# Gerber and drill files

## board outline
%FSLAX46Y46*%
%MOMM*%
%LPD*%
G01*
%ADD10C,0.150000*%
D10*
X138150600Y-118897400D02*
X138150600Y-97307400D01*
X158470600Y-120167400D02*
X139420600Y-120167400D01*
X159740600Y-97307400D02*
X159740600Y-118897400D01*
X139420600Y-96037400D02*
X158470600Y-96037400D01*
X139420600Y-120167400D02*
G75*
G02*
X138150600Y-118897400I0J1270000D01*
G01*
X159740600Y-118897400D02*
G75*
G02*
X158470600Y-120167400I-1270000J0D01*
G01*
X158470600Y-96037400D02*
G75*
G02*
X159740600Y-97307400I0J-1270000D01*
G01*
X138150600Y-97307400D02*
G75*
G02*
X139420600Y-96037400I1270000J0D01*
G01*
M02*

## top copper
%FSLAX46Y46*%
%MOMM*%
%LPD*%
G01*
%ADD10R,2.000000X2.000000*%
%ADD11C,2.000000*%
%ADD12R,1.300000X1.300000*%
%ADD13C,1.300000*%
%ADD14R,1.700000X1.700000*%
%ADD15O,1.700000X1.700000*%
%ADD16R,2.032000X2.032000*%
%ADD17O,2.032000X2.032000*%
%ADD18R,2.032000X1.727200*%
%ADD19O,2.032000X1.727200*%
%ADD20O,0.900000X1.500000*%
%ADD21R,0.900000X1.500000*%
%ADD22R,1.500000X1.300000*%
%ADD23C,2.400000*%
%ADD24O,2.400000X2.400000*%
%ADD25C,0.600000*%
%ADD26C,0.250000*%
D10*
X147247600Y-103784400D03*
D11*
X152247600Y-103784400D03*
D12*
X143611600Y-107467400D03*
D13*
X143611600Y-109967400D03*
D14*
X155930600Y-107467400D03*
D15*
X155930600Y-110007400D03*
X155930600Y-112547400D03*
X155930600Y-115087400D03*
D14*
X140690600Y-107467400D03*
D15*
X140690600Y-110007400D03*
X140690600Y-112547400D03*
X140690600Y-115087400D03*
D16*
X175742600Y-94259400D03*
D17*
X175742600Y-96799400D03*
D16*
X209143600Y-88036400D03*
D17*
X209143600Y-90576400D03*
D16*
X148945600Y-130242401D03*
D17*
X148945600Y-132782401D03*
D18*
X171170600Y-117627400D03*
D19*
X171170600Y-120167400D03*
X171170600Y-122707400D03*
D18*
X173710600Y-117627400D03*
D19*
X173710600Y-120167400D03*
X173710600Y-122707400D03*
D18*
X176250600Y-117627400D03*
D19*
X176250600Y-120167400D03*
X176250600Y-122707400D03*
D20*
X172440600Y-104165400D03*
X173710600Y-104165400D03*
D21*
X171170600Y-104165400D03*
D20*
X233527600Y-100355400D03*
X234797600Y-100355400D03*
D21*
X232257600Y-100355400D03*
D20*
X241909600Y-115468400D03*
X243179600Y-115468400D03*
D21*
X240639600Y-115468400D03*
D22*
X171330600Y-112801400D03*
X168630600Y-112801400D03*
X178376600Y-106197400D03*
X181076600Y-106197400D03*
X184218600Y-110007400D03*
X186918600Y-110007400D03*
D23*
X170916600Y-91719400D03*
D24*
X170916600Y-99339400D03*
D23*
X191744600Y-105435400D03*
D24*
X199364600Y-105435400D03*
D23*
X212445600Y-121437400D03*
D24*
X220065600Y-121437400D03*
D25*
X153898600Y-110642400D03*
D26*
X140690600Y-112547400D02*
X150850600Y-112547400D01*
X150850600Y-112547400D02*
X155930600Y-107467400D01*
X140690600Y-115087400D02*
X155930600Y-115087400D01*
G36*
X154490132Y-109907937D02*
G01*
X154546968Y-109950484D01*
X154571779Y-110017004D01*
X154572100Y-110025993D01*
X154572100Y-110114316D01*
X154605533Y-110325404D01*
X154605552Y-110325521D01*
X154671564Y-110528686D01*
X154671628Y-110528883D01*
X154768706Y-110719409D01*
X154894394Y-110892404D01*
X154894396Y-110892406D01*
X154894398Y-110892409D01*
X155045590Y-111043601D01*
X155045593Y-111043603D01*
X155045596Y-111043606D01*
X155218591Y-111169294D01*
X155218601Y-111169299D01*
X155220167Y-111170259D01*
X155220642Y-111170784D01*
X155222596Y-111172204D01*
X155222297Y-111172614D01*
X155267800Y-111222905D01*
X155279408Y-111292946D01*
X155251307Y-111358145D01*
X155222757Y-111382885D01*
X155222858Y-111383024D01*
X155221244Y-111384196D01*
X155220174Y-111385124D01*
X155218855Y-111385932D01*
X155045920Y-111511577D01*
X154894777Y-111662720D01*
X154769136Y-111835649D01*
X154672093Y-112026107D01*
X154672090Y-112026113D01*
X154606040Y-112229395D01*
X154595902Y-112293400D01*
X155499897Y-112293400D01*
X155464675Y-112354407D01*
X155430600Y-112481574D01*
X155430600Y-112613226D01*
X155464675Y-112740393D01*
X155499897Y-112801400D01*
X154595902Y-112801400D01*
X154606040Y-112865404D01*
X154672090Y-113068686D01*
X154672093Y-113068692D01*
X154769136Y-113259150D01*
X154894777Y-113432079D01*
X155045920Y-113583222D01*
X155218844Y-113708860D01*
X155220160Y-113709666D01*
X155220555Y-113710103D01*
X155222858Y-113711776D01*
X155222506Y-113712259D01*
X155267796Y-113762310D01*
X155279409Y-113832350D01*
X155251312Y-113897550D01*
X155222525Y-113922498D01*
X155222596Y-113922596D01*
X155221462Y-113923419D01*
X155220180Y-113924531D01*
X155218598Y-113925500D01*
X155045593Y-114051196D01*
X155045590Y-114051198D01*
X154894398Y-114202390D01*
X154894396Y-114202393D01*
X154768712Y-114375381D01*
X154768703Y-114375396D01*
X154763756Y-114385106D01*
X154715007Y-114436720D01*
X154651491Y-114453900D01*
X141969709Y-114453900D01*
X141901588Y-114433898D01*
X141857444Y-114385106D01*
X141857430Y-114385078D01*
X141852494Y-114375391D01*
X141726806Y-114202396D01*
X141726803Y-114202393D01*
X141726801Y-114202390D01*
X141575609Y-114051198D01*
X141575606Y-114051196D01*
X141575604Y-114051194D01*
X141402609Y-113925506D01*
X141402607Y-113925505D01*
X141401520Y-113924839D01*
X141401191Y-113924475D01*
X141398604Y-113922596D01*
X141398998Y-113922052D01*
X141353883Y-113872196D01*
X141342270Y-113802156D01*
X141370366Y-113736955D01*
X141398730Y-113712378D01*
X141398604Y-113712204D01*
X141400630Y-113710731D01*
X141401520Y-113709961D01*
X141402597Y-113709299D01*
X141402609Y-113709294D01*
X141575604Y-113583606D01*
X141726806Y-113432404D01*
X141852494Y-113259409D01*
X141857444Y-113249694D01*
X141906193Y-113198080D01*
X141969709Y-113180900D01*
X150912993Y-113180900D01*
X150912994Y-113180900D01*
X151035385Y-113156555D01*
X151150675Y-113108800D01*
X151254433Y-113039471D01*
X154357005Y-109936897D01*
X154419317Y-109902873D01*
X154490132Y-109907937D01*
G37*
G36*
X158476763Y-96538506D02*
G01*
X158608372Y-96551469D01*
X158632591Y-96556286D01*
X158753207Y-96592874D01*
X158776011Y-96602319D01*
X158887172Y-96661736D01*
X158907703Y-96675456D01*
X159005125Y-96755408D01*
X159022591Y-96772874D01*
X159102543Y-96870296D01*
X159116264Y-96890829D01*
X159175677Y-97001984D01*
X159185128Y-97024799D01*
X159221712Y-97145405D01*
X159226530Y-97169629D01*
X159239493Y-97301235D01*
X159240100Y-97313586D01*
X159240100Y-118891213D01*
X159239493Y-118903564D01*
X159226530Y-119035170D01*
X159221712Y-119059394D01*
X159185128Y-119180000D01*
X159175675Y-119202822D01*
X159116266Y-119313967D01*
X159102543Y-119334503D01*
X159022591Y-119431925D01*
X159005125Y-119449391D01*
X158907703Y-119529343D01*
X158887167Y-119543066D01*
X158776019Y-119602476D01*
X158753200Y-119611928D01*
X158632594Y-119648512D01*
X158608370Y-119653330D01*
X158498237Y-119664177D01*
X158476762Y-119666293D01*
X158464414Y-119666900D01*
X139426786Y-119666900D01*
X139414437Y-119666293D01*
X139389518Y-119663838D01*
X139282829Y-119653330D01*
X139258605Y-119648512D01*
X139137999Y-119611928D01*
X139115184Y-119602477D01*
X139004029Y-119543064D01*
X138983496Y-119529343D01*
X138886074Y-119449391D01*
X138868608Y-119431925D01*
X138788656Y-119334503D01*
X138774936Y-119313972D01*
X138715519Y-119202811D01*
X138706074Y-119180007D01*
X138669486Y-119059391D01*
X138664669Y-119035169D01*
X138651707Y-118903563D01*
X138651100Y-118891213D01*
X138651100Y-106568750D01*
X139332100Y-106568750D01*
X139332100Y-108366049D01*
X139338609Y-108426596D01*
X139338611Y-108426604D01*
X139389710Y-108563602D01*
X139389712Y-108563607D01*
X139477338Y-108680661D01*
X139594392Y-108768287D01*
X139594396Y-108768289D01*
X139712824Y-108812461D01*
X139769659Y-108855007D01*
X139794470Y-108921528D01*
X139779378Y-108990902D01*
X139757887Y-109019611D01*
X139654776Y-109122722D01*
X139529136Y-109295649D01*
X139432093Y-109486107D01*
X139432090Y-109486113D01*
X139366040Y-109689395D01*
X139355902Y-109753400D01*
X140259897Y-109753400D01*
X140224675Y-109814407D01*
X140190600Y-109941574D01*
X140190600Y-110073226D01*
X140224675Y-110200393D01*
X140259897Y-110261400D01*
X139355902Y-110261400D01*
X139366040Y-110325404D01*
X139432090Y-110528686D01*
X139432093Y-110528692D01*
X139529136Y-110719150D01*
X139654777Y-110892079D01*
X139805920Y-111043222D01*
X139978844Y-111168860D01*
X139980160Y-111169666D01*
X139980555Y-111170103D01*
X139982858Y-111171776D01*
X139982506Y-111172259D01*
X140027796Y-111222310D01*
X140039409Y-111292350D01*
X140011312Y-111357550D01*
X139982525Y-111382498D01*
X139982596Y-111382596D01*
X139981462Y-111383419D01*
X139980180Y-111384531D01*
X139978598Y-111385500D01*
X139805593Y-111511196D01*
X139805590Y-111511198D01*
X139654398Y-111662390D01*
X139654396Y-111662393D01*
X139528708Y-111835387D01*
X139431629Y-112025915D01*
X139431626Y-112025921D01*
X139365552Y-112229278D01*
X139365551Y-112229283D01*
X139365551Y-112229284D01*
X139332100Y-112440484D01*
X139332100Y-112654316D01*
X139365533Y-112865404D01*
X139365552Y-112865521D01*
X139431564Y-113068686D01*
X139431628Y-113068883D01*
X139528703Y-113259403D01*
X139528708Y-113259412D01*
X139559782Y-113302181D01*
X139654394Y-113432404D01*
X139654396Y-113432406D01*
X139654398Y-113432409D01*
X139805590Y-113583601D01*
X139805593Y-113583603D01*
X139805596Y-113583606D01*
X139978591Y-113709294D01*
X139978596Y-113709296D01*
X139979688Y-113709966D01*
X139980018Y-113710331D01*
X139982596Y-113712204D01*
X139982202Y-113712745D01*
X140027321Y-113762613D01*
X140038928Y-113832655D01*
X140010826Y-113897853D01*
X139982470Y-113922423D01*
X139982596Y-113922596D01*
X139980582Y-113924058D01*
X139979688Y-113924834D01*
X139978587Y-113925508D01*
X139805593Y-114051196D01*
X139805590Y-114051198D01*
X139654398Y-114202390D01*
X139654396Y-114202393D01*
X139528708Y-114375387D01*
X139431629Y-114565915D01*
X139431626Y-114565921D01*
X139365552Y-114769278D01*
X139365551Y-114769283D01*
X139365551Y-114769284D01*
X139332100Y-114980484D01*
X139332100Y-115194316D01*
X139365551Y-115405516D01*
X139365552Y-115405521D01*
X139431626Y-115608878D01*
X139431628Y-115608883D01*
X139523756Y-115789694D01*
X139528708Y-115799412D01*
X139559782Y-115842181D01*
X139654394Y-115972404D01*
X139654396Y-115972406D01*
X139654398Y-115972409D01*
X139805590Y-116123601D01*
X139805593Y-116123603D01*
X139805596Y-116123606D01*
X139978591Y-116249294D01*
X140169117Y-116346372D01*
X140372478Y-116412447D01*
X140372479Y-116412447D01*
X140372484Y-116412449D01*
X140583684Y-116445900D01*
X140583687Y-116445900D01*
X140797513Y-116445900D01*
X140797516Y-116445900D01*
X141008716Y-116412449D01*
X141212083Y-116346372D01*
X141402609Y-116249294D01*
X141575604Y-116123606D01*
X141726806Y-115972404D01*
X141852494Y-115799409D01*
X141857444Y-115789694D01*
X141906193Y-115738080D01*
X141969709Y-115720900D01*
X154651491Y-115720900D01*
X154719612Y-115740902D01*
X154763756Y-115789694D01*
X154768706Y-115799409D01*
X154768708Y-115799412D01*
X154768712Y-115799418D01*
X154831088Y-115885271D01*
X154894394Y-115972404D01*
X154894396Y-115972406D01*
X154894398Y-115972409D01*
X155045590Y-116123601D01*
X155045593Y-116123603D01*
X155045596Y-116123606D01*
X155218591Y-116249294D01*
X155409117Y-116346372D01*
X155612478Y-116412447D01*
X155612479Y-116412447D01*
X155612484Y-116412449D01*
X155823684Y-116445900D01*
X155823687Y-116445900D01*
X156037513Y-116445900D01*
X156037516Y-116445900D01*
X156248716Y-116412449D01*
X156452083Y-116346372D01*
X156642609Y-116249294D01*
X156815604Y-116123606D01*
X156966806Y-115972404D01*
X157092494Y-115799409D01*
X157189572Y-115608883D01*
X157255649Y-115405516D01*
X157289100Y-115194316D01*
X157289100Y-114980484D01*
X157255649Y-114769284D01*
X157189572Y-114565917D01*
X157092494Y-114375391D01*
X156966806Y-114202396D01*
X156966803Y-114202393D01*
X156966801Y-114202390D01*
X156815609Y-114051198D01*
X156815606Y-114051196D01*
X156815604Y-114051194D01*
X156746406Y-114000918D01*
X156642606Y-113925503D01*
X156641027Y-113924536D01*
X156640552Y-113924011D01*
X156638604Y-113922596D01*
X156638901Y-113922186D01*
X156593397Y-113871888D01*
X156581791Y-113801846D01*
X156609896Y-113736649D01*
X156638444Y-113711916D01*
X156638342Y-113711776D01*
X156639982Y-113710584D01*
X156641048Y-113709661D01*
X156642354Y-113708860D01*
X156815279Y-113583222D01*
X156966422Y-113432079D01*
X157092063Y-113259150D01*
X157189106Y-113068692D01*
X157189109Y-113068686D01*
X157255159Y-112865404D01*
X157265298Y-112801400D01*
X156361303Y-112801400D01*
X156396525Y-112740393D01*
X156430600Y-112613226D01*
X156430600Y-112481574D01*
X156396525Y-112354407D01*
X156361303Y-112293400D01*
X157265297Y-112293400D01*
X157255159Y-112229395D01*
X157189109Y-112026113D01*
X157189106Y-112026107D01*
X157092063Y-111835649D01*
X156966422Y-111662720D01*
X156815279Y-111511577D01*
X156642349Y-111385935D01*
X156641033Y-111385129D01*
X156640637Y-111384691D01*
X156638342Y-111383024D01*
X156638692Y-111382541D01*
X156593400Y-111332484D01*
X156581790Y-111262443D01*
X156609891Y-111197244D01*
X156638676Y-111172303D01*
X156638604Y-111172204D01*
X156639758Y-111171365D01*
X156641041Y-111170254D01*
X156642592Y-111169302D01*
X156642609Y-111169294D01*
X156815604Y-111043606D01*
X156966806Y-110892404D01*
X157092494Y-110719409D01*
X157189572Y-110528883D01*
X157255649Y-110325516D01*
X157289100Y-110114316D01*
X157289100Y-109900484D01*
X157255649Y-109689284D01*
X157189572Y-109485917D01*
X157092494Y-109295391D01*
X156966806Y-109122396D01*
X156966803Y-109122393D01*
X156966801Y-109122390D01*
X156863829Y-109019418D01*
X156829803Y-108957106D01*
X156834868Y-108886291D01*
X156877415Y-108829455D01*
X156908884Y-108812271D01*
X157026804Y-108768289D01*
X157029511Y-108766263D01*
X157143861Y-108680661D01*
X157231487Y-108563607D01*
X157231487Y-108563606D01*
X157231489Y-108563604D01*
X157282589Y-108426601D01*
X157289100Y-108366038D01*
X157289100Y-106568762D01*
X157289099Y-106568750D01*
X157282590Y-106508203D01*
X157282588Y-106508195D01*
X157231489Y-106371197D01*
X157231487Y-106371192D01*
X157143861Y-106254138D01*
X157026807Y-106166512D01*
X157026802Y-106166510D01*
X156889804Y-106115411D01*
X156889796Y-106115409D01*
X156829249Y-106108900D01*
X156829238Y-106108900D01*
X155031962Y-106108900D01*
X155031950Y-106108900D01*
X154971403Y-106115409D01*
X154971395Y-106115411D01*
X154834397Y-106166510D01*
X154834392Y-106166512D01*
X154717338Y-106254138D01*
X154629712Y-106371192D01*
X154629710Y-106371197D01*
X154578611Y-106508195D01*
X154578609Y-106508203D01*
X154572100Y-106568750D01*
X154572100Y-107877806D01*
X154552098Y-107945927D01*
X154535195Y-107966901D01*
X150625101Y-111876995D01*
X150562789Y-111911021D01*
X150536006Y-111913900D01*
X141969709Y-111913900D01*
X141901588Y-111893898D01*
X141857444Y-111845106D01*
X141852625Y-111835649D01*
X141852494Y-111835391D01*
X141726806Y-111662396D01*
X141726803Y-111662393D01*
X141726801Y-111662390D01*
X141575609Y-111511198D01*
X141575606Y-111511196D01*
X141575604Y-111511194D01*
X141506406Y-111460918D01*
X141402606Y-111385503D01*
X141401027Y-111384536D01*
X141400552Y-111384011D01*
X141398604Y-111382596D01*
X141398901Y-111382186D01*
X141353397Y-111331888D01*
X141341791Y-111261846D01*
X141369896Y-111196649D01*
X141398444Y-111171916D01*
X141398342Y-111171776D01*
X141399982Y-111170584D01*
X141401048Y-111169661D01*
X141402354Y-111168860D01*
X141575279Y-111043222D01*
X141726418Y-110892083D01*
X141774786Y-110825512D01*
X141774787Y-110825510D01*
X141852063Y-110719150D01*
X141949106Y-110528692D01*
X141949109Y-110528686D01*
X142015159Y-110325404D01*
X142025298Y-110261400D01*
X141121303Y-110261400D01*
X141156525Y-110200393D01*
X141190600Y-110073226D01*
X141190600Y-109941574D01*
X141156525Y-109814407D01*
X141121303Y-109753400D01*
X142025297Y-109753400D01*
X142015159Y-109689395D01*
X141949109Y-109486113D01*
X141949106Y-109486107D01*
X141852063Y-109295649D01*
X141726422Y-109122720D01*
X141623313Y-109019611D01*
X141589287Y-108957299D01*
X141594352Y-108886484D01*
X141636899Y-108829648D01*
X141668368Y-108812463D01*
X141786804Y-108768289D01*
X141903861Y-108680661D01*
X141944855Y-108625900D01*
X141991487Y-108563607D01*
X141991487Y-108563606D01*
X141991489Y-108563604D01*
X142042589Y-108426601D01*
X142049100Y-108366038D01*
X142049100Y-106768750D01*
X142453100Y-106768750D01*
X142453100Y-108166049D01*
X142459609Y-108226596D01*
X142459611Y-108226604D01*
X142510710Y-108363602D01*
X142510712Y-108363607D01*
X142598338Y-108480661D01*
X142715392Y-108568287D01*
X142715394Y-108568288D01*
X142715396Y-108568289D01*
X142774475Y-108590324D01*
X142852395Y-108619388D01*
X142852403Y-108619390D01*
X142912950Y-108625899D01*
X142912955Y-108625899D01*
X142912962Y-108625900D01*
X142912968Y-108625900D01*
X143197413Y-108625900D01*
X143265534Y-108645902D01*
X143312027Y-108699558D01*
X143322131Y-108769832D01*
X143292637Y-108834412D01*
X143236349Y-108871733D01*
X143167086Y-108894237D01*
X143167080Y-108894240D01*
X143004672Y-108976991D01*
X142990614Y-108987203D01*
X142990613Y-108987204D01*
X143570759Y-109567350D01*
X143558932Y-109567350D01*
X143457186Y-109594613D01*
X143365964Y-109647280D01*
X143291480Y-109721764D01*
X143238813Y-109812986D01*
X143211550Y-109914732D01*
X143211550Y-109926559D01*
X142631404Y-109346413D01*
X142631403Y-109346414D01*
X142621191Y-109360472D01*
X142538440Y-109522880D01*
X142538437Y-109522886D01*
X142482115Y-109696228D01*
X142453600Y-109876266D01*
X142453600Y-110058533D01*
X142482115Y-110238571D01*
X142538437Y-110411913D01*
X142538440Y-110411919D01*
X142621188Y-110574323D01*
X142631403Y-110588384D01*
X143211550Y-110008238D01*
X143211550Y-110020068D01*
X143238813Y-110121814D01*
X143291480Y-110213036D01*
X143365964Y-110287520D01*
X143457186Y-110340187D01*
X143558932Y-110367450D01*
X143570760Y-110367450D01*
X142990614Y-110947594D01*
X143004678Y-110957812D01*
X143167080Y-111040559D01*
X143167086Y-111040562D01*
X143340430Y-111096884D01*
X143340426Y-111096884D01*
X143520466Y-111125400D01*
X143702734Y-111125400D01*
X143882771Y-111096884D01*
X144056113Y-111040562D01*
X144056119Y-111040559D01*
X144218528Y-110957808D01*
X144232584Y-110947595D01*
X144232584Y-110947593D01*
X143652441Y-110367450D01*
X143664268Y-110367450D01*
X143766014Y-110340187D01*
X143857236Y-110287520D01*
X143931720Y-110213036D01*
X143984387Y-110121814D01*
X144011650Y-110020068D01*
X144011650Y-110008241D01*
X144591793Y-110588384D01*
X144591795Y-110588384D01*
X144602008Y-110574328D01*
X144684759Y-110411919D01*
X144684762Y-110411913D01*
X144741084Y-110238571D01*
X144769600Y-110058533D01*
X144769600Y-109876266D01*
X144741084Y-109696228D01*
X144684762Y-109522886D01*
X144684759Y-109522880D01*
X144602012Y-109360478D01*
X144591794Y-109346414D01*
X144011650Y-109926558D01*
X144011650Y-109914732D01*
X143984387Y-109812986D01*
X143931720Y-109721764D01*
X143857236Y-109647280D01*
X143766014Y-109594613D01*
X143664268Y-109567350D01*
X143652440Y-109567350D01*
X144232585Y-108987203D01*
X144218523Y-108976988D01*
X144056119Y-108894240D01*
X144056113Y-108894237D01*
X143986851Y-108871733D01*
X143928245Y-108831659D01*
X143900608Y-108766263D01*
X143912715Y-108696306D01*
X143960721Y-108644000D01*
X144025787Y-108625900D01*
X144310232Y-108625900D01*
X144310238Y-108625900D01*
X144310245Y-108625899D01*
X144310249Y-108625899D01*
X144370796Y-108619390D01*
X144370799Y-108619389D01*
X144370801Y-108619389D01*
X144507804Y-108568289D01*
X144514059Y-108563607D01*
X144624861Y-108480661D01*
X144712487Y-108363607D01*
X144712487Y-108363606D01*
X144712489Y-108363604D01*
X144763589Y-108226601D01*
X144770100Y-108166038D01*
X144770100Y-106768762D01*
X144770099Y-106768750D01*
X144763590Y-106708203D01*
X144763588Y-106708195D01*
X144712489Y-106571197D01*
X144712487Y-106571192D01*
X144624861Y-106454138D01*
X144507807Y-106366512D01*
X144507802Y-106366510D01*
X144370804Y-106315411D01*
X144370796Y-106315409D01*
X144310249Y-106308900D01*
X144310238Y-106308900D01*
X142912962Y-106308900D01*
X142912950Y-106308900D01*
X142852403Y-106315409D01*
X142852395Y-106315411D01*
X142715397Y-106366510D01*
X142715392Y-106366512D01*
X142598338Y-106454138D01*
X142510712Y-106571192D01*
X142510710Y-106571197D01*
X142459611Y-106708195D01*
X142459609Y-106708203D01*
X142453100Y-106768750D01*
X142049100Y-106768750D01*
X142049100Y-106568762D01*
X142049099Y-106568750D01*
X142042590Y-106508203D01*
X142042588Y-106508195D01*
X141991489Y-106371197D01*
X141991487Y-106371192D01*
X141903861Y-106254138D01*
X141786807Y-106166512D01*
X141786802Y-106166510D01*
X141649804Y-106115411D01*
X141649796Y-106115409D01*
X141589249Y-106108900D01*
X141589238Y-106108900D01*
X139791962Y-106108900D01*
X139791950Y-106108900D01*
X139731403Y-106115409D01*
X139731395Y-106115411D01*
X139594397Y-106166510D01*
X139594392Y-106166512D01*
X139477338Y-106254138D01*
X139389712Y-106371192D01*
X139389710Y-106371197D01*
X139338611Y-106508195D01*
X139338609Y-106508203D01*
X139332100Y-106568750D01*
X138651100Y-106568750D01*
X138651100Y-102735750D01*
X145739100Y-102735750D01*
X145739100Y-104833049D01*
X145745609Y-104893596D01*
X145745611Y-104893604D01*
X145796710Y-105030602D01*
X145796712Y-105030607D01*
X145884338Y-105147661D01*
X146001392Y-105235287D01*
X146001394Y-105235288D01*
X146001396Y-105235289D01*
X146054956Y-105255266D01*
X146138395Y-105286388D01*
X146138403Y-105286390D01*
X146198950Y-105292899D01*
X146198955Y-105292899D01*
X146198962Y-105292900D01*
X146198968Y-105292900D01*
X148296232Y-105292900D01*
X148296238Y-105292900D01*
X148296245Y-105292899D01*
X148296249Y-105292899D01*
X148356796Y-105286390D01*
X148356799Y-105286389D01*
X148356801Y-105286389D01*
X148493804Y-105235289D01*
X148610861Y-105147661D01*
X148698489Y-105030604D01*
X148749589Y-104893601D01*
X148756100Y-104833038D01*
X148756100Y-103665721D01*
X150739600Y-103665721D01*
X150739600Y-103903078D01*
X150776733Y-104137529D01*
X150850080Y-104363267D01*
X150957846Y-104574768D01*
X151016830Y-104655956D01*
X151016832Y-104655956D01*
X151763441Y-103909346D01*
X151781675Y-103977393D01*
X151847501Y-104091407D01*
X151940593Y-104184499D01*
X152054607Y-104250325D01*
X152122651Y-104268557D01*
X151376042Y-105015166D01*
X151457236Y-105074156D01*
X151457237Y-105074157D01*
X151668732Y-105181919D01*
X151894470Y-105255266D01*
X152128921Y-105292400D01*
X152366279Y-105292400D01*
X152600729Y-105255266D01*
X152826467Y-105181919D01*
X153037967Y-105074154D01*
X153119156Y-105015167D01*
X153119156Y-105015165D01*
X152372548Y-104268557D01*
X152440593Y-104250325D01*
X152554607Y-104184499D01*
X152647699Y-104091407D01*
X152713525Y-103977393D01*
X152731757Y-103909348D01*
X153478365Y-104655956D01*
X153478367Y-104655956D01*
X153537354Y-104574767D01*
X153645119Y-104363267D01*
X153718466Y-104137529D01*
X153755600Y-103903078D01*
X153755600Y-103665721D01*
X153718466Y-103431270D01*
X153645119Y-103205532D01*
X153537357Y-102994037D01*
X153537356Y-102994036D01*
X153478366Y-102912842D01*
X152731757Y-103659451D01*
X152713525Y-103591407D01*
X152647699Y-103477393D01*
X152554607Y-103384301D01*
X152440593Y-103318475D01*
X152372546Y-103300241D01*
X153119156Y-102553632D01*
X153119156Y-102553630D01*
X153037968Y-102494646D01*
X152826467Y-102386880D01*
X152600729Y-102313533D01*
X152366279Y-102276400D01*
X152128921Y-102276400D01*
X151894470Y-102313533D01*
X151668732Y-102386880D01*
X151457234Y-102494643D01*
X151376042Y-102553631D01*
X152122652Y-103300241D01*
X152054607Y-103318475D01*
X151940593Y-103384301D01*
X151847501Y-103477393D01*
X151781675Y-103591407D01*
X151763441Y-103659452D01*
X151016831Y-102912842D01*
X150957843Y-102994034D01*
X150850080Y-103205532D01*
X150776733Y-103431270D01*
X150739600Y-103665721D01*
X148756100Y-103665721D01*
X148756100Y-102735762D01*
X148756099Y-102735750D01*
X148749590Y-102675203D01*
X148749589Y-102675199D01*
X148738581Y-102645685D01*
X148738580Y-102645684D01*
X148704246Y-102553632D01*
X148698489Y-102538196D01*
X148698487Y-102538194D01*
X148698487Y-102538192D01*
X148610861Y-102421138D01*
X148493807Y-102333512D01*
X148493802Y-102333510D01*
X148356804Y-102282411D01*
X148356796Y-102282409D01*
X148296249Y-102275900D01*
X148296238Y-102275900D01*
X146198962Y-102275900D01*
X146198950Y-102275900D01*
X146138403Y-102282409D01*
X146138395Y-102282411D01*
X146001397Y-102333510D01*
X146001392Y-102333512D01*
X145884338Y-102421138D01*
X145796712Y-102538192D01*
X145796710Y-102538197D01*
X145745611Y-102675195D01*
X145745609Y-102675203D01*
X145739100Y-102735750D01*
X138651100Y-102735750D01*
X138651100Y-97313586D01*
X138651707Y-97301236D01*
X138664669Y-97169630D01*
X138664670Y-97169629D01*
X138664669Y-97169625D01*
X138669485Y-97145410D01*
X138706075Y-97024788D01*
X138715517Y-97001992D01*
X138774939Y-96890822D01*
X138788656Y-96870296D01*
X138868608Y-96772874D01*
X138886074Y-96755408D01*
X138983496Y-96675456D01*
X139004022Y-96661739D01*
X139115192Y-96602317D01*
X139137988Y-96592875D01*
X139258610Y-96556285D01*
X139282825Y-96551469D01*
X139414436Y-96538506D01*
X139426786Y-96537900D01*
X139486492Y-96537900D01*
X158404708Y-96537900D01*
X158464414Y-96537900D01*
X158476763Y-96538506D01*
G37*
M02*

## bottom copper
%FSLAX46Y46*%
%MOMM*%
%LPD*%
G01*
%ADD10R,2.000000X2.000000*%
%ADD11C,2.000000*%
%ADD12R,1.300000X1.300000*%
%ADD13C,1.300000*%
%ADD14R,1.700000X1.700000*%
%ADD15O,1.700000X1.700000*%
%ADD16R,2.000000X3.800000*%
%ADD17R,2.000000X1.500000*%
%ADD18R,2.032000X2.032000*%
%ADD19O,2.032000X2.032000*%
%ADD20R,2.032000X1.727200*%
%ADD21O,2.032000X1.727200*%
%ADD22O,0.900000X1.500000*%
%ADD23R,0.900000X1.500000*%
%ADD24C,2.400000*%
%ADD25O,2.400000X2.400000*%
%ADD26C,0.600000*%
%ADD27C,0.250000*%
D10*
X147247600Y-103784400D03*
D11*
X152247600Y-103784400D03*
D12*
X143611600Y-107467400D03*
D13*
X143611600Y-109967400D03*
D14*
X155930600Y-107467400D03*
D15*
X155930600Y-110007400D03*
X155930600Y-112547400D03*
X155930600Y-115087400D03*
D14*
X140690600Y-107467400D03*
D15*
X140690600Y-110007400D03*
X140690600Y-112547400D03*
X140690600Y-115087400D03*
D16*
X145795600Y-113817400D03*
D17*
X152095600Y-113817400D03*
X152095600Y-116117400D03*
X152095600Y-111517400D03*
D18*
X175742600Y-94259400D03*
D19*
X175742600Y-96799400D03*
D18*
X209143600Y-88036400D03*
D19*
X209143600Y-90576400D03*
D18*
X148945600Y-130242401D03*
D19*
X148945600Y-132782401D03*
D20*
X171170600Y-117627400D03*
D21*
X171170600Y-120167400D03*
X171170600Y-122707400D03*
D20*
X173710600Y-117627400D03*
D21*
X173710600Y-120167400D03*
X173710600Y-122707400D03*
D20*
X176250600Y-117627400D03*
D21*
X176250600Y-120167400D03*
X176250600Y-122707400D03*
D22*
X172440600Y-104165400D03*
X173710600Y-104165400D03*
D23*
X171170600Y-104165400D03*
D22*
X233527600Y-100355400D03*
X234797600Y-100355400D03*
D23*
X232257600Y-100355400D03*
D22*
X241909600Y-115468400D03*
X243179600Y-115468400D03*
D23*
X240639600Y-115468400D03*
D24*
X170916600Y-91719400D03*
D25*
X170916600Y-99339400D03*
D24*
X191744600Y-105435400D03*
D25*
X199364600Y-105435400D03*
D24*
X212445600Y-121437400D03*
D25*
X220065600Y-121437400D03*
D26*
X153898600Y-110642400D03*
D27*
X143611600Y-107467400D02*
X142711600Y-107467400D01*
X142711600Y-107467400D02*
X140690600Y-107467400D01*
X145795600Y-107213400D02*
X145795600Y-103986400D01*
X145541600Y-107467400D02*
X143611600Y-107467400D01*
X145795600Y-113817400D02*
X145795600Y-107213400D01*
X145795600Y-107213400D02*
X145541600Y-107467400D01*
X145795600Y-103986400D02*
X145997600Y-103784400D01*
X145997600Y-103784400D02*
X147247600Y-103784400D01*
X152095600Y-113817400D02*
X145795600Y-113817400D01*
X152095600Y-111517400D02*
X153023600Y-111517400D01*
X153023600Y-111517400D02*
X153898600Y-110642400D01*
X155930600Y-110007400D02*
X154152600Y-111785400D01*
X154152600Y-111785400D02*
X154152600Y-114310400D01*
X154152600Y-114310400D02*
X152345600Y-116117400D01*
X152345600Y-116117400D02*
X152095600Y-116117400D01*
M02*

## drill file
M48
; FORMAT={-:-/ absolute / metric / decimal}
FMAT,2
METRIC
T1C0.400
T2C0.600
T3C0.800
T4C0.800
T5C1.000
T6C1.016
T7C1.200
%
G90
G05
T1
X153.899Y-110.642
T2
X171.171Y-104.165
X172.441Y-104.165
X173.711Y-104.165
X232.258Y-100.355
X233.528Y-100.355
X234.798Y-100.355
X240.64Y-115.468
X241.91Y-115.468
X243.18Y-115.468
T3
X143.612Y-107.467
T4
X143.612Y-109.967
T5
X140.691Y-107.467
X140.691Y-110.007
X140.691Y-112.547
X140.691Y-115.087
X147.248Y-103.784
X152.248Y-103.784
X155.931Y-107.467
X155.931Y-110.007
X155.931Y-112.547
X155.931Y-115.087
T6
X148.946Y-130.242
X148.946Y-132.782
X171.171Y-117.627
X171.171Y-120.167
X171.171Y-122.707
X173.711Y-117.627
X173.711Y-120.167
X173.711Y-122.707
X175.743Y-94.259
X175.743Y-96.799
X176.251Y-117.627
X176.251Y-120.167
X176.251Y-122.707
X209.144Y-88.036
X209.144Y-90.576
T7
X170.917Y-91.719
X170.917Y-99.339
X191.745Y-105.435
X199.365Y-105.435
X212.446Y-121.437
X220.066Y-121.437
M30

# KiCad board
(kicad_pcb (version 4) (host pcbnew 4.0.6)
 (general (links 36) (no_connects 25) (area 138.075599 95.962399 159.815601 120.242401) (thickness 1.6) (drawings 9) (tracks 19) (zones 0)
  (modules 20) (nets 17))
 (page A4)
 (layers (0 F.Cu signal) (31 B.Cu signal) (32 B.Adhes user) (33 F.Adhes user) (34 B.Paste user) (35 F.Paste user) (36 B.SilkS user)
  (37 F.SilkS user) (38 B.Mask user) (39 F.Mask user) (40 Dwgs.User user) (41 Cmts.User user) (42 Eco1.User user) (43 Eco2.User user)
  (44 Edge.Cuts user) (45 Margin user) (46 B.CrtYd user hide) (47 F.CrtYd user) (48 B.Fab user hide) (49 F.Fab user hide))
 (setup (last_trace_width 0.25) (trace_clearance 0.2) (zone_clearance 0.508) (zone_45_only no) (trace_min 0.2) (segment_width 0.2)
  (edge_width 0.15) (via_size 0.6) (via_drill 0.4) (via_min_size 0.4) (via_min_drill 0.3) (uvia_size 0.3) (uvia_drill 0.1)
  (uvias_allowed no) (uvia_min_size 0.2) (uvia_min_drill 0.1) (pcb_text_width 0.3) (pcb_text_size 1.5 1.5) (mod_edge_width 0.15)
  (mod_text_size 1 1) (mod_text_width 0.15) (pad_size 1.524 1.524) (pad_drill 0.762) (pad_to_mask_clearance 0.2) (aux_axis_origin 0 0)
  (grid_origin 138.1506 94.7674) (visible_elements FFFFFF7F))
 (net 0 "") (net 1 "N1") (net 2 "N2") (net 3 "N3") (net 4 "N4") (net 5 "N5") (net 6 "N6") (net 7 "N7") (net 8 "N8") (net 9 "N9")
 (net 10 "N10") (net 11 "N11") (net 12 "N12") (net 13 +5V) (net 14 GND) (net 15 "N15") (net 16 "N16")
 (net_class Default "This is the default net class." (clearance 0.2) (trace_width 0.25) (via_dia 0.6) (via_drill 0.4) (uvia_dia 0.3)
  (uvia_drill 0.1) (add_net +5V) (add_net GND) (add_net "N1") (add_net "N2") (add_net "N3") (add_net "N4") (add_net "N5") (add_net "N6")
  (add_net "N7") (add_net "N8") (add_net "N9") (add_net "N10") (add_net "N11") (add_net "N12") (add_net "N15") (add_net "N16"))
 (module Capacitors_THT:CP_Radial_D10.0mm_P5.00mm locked (layer F.Cu) (at 147.2476 103.7844)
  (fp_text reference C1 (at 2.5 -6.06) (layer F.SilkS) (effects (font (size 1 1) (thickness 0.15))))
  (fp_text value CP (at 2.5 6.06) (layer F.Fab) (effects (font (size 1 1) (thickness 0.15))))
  (pad 1 thru_hole rect (at 0 0) (size 2 2) (drill 1) (layers *.Cu *.Mask) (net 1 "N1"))
  (pad 2 thru_hole circle (at 5 0) (size 2 2) (drill 1) (layers *.Cu *.Mask) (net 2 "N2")))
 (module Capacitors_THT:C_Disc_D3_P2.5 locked (layer F.Cu) (at 143.6116 107.4674 270)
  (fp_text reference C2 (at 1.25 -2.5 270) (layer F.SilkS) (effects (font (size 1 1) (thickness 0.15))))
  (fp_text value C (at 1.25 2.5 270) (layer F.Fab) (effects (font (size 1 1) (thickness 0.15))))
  (pad 1 thru_hole rect (at 0 0 270) (size 1.3 1.3) (drill 0.8) (layers *.Cu *.Mask) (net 1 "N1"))
  (pad 2 thru_hole circle (at 2.5 0 270) (size 1.3 1.3) (drill 0.8001) (layers *.Cu *.Mask) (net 2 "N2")))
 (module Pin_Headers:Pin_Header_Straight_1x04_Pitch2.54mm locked (layer F.Cu) (at 155.9306 107.4674)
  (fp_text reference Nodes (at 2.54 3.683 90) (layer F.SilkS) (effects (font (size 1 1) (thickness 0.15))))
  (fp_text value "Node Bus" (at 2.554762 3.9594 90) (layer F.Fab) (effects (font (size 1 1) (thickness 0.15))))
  (pad 1 thru_hole rect (at 0 0) (size 1.7 1.7) (drill 1) (layers *.Cu *.Mask) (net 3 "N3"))
  (pad 2 thru_hole oval (at 0 2.54) (size 1.7 1.7) (drill 1) (layers *.Cu *.Mask) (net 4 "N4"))
  (pad 3 thru_hole oval (at 0 5.08) (size 1.7 1.7) (drill 1) (layers *.Cu *.Mask) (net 2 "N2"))
  (pad 4 thru_hole oval (at 0 7.62) (size 1.7 1.7) (drill 1) (layers *.Cu *.Mask) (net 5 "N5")))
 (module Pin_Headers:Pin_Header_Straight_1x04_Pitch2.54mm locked (layer F.Cu) (at 140.6906 107.4674)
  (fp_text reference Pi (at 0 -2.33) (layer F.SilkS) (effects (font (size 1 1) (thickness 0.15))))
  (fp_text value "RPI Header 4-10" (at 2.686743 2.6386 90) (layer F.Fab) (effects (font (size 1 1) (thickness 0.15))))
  (pad 1 thru_hole rect (at 0 0) (size 1.7 1.7) (drill 1) (layers *.Cu *.Mask) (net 1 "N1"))
  (pad 2 thru_hole oval (at 0 2.54) (size 1.7 1.7) (drill 1) (layers *.Cu *.Mask) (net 2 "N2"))
  (pad 3 thru_hole oval (at 0 5.08) (size 1.7 1.7) (drill 1) (layers *.Cu *.Mask) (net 3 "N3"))
  (pad 4 thru_hole oval (at 0 7.62) (size 1.7 1.7) (drill 1) (layers *.Cu *.Mask) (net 5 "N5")))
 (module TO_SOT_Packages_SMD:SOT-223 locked (layer B.Cu) (at 148.9456 113.8174 180)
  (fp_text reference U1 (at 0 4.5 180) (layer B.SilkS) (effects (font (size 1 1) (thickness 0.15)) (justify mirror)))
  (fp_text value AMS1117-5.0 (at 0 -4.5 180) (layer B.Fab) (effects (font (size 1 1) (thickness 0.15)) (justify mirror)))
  (pad 4 smd rect (at 3.15 0 180) (size 2 3.8) (layers B.Cu B.Paste B.Mask) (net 1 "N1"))
  (pad 2 smd rect (at -3.15 0 180) (size 2 1.5) (layers B.Cu B.Paste B.Mask) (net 1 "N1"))
  (pad 3 smd rect (at -3.15 -2.3 180) (size 2 1.5) (layers B.Cu B.Paste B.Mask) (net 4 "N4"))
  (pad 1 smd rect (at -3.15 2.3 180) (size 2 1.5) (layers B.Cu B.Paste B.Mask) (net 2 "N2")))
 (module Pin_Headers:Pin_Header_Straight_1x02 (layer F.Cu) (at 175.7426 94.2594)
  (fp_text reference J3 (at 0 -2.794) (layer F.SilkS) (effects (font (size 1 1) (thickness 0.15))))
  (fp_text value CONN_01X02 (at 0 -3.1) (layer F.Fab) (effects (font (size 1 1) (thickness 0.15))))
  (pad 1 thru_hole rect (at 0 0) (size 2.032 2.032) (drill 1.016) (layers *.Cu *.Mask) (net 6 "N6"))
  (pad 2 thru_hole oval (at 0 2.54) (size 2.032 2.032) (drill 1.016) (layers *.Cu *.Mask) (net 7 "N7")))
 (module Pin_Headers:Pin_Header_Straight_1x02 (layer F.Cu) (at 209.1436 88.0364)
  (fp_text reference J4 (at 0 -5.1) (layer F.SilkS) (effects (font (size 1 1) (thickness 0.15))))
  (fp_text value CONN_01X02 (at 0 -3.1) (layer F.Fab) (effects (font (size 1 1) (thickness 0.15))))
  (pad 1 thru_hole rect (at 0 0) (size 2.032 2.032) (drill 1.016) (layers *.Cu *.Mask) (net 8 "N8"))
  (pad 2 thru_hole oval (at 0 2.54) (size 2.032 2.032) (drill 1.016) (layers *.Cu *.Mask) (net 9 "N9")))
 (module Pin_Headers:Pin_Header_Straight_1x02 (layer F.Cu) (at 148.9456 130.242401)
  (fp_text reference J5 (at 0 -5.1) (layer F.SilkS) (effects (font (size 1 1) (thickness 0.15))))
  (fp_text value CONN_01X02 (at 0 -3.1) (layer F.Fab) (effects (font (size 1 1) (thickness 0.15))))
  (pad 1 thru_hole rect (at 0 0) (size 2.032 2.032) (drill 1.016) (layers *.Cu *.Mask) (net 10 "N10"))
  (pad 2 thru_hole oval (at 0 2.54) (size 2.032 2.032) (drill 1.016) (layers *.Cu *.Mask) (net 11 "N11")))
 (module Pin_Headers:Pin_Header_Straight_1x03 (layer F.Cu) (at 171.1706 117.6274)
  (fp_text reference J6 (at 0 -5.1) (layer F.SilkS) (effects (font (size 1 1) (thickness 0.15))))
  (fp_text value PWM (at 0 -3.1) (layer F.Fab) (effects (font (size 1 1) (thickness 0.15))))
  (pad 1 thru_hole rect (at 0 0) (size 2.032 1.7272) (drill 1.016) (layers *.Cu *.Mask) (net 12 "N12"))
  (pad 2 thru_hole oval (at 0 2.54) (size 2.032 1.7272) (drill 1.016) (layers *.Cu *.Mask) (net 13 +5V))
  (pad 3 thru_hole oval (at 0 5.08) (size 2.032 1.7272) (drill 1.016) (layers *.Cu *.Mask) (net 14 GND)))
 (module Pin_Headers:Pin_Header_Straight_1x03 (layer F.Cu) (at 173.7106 117.6274)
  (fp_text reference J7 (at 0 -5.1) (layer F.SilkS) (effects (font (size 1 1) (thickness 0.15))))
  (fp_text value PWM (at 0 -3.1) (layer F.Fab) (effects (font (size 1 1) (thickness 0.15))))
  (pad 1 thru_hole rect (at 0 0) (size 2.032 1.7272) (drill 1.016) (layers *.Cu *.Mask) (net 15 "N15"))
  (pad 2 thru_hole oval (at 0 2.54) (size 2.032 1.7272) (drill 1.016) (layers *.Cu *.Mask) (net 13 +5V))
  (pad 3 thru_hole oval (at 0 5.08) (size 2.032 1.7272) (drill 1.016) (layers *.Cu *.Mask) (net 14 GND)))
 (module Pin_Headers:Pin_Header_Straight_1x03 (layer F.Cu) (at 176.2506 117.6274)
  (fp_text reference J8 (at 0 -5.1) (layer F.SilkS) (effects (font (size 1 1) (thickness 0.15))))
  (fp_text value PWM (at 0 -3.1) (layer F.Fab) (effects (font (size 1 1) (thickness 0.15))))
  (pad 1 thru_hole rect (at 0 0) (size 2.032 1.7272) (drill 1.016) (layers *.Cu *.Mask) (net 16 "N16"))
  (pad 2 thru_hole oval (at 0 2.54) (size 2.032 1.7272) (drill 1.016) (layers *.Cu *.Mask) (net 13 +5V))
  (pad 3 thru_hole oval (at 0 5.08) (size 2.032 1.7272) (drill 1.016) (layers *.Cu *.Mask) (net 14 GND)))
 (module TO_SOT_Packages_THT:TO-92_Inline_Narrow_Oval (layer F.Cu) (at 171.1706 104.1654)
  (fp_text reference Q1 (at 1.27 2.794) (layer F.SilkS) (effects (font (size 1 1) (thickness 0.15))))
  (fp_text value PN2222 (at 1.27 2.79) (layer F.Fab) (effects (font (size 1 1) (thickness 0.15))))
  (pad 2 thru_hole oval (at 1.27 0 180) (size 0.9 1.5) (drill 0.6) (layers *.Cu *.Mask) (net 12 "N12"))
  (pad 3 thru_hole oval (at 2.54 0 180) (size 0.9 1.5) (drill 0.6) (layers *.Cu *.Mask) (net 7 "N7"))
  (pad 1 thru_hole rect (at 0 0 180) (size 0.9 1.5) (drill 0.6) (layers *.Cu *.Mask) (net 14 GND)))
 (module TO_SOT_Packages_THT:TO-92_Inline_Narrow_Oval (layer F.Cu) (at 232.2576 100.3554)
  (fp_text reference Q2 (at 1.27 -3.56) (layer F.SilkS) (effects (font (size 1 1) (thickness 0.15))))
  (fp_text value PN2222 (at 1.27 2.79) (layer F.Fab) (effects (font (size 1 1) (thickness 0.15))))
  (pad 2 thru_hole oval (at 1.27 0 180) (size 0.9 1.5) (drill 0.6) (layers *.Cu *.Mask) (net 15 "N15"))
  (pad 3 thru_hole oval (at 2.54 0 180) (size 0.9 1.5) (drill 0.6) (layers *.Cu *.Mask) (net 9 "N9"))
  (pad 1 thru_hole rect (at 0 0 180) (size 0.9 1.5) (drill 0.6) (layers *.Cu *.Mask) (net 14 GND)))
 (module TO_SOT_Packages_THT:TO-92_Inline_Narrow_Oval (layer F.Cu) (at 240.6396 115.4684)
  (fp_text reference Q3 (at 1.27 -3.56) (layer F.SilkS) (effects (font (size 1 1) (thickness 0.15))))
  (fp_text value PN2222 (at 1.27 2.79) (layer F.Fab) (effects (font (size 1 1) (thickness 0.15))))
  (pad 2 thru_hole oval (at 1.27 0 180) (size 0.9 1.5) (drill 0.6) (layers *.Cu *.Mask) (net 16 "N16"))
  (pad 3 thru_hole oval (at 2.54 0 180) (size 0.9 1.5) (drill 0.6) (layers *.Cu *.Mask) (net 11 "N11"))
  (pad 1 thru_hole rect (at 0 0 180) (size 0.9 1.5) (drill 0.6) (layers *.Cu *.Mask) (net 14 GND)))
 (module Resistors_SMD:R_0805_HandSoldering (layer F.Cu) (at 169.9806 112.8014 180)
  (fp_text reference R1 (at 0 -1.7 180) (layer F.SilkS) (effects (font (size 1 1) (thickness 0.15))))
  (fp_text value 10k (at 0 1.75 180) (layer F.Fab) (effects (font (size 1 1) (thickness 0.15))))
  (pad 1 smd rect (at -1.35 0 180) (size 1.5 1.3) (layers F.Cu F.Paste F.Mask) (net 12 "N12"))
  (pad 2 smd rect (at 1.35 0 180) (size 1.5 1.3) (layers F.Cu F.Paste F.Mask) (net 14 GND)))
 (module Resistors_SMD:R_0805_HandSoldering (layer F.Cu) (at 179.7266 106.1974)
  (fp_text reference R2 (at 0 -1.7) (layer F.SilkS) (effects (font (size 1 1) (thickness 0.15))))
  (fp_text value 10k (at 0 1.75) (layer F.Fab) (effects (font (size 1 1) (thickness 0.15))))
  (pad 1 smd rect (at -1.35 0) (size 1.5 1.3) (layers F.Cu F.Paste F.Mask) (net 15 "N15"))
  (pad 2 smd rect (at 1.35 0) (size 1.5 1.3) (layers F.Cu F.Paste F.Mask) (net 14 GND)))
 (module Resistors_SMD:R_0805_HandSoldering (layer F.Cu) (at 185.5686 110.0074)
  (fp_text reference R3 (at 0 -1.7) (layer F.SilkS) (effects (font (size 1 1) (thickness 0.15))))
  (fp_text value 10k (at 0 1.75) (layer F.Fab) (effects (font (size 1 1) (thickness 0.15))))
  (pad 1 smd rect (at -1.35 0) (size 1.5 1.3) (layers F.Cu F.Paste F.Mask) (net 16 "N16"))
  (pad 2 smd rect (at 1.35 0) (size 1.5 1.3) (layers F.Cu F.Paste F.Mask) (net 14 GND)))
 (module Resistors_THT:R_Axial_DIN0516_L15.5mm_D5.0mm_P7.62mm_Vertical (layer F.Cu) (at 170.9166 91.7194 270)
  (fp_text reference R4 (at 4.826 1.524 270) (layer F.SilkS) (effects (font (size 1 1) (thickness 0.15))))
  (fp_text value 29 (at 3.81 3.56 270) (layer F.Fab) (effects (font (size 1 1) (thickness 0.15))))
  (pad 1 thru_hole circle (at 0 0 270) (size 2.4 2.4) (drill 1.2) (layers *.Cu *.Mask) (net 6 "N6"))
  (pad 2 thru_hole oval (at 7.62 0 270) (size 2.4 2.4) (drill 1.2) (layers *.Cu *.Mask) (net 13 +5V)))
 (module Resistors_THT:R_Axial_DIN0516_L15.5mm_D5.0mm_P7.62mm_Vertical (layer F.Cu) (at 191.7446 105.4354)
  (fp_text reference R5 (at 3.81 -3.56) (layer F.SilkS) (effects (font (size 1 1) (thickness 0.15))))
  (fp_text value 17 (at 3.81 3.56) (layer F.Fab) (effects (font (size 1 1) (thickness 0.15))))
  (pad 1 thru_hole circle (at 0 0) (size 2.4 2.4) (drill 1.2) (layers *.Cu *.Mask) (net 8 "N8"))
  (pad 2 thru_hole oval (at 7.62 0) (size 2.4 2.4) (drill 1.2) (layers *.Cu *.Mask) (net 13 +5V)))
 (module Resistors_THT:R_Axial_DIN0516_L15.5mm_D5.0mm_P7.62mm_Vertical (layer F.Cu) (at 212.4456 121.4374)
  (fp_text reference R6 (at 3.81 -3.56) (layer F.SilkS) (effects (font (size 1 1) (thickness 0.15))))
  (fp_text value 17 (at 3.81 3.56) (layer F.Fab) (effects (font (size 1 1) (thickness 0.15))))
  (pad 1 thru_hole circle (at 0 0) (size 2.4 2.4) (drill 1.2) (layers *.Cu *.Mask) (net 10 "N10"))
  (pad 2 thru_hole oval (at 7.62 0) (size 2.4 2.4) (drill 1.2) (layers *.Cu *.Mask) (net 13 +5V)))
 (gr_line (start 138.1506 118.8974) (end 138.1506 97.3074) (layer Edge.Cuts) (width 0.15))
 (gr_line (start 158.4706 120.1674) (end 139.4206 120.1674) (layer Edge.Cuts) (width 0.15))
 (gr_line (start 159.7406 97.3074) (end 159.7406 118.8974) (layer Edge.Cuts) (width 0.15))
 (gr_line (start 139.4206 96.0374) (end 158.4706 96.0374) (layer Edge.Cuts) (width 0.15))
 (gr_arc (start 139.4206 118.8974) (end 139.4206 120.1674) (angle 90) (layer Edge.Cuts) (width 0.15))
 (gr_arc (start 158.4706 118.8974) (end 159.7406 118.8974) (angle 90) (layer Edge.Cuts) (width 0.15))
 (gr_arc (start 158.4706 97.3074) (end 158.4706 96.0374) (angle 90) (layer Edge.Cuts) (width 0.15))
 (gr_arc (start 139.4206 97.3074) (end 138.1506 97.3074) (angle 90) (layer Edge.Cuts) (width 0.15))
 (segment (start 143.6116 107.4674) (end 142.7116 107.4674) (width 0.25) (layer B.Cu) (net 1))
 (segment (start 142.7116 107.4674) (end 140.6906 107.4674) (width 0.25) (layer B.Cu) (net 1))
 (segment (start 145.7956 107.2134) (end 145.7956 103.9864) (width 0.25) (layer B.Cu) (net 1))
 (segment (start 145.5416 107.4674) (end 143.6116 107.4674) (width 0.25) (layer B.Cu) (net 1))
 (segment (start 145.7956 113.8174) (end 145.7956 107.2134) (width 0.25) (layer B.Cu) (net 1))
 (segment (start 145.7956 107.2134) (end 145.5416 107.4674) (width 0.25) (layer B.Cu) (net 1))
 (segment (start 145.7956 103.9864) (end 145.9976 103.7844) (width 0.25) (layer B.Cu) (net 1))
 (segment (start 145.9976 103.7844) (end 147.2476 103.7844) (width 0.25) (layer B.Cu) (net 1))
 (segment (start 152.0956 113.8174) (end 145.7956 113.8174) (width 0.25) (layer B.Cu) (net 1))
 (segment (start 152.0956 111.5174) (end 153.0236 111.5174) (width 0.25) (layer B.Cu) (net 2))
 (segment (start 153.0236 111.5174) (end 153.8986 110.6424) (width 0.25) (layer B.Cu) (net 2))
 (via (at 153.8986 110.6424) (size 0.6) (drill 0.4) (layers F.Cu B.Cu) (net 2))
 (segment (start 140.6906 112.5474) (end 150.8506 112.5474) (width 0.25) (layer F.Cu) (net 3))
 (segment (start 150.8506 112.5474) (end 155.9306 107.4674) (width 0.25) (layer F.Cu) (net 3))
 (segment (start 155.9306 110.0074) (end 154.1526 111.7854) (width 0.25) (layer B.Cu) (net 4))
 (segment (start 154.1526 111.7854) (end 154.1526 114.3104) (width 0.25) (layer B.Cu) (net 4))
 (segment (start 154.1526 114.3104) (end 152.3456 116.1174) (width 0.25) (layer B.Cu) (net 4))
 (segment (start 152.3456 116.1174) (end 152.0956 116.1174) (width 0.25) (layer B.Cu) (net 4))
 (segment (start 140.6906 115.0874) (end 155.9306 115.0874) (width 0.25) (layer F.Cu) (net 5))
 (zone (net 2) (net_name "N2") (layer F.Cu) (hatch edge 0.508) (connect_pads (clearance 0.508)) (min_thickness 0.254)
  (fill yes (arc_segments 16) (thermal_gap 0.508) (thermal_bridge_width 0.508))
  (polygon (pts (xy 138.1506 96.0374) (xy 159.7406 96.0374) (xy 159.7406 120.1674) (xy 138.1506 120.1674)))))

